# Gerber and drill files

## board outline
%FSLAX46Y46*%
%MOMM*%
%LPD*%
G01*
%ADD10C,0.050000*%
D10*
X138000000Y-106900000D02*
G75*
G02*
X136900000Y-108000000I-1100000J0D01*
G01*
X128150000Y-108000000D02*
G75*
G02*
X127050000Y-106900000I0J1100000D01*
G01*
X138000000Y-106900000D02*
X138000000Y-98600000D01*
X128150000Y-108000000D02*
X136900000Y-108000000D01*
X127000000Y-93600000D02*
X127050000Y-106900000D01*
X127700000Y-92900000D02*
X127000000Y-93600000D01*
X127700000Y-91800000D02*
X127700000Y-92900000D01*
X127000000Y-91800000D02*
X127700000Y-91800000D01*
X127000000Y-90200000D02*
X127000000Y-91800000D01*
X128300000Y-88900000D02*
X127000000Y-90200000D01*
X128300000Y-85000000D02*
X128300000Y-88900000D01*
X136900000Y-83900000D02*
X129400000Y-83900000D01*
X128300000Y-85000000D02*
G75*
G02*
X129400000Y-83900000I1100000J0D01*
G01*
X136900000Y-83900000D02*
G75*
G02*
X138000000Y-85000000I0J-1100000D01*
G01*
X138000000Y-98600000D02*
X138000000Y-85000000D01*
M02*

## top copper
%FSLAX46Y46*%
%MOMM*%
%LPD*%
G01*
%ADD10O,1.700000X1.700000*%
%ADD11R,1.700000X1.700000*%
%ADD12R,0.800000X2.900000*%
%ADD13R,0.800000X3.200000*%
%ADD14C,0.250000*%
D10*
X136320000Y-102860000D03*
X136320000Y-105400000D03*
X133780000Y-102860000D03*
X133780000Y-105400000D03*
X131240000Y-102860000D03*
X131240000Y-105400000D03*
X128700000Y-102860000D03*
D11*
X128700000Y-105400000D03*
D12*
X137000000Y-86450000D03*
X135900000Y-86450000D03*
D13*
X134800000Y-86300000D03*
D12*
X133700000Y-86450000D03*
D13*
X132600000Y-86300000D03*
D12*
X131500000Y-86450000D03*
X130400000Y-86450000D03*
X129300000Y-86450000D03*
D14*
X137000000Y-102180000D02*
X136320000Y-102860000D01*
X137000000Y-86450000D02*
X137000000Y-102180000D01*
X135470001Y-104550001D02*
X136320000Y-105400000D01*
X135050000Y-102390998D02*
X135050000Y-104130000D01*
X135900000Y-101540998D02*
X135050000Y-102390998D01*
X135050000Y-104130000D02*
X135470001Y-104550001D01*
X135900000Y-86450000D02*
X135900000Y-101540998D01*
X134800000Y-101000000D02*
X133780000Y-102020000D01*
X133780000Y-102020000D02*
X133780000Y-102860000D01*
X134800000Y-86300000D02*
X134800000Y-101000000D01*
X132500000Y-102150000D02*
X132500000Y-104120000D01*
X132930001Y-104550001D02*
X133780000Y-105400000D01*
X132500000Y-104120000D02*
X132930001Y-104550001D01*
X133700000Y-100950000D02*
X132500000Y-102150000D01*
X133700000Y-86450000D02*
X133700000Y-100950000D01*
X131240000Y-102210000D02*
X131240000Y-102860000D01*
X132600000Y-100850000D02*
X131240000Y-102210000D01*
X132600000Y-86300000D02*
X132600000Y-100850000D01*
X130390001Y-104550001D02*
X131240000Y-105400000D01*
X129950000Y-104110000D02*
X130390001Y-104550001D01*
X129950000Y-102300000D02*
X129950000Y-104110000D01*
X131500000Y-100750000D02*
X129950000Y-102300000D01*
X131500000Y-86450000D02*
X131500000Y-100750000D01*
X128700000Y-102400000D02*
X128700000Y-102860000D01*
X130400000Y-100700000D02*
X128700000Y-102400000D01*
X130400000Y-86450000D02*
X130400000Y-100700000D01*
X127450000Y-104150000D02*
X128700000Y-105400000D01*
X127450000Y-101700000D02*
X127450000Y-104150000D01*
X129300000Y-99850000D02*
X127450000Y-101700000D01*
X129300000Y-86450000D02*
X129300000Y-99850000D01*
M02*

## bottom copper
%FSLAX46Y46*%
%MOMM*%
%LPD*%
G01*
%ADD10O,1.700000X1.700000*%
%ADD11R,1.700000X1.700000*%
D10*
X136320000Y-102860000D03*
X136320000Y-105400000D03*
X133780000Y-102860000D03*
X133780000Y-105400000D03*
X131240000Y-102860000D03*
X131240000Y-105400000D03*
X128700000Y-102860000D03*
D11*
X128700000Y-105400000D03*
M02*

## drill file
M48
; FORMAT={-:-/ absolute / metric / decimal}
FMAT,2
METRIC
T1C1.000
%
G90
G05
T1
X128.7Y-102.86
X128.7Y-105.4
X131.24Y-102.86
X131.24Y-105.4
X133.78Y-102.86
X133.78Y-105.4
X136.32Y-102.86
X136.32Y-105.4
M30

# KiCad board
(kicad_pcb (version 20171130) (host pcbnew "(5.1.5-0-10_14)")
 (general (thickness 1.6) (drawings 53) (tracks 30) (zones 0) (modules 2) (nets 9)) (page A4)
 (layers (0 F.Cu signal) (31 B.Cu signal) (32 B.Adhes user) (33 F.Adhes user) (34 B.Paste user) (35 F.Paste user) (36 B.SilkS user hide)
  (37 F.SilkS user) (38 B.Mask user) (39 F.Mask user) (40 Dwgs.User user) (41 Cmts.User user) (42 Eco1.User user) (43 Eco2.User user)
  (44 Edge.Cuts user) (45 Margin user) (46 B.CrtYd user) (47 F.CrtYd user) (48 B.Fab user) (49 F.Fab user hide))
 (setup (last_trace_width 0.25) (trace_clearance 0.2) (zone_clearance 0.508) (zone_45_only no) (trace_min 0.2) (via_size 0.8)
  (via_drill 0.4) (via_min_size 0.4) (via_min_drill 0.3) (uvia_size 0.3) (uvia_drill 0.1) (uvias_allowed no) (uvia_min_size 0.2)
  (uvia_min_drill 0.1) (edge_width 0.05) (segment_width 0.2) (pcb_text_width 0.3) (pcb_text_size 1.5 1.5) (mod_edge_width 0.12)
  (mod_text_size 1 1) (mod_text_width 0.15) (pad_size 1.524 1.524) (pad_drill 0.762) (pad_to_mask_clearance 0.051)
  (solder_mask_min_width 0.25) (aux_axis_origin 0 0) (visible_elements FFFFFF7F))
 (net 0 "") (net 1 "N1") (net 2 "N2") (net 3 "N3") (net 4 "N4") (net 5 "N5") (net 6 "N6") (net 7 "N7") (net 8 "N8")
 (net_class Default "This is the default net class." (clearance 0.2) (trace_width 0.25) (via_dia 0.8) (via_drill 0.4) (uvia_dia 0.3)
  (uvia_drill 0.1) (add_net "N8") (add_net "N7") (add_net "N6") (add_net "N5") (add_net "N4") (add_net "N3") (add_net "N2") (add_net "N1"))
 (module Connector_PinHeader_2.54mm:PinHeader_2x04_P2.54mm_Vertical (layer F.Cu) (at 128.7 105.4 90)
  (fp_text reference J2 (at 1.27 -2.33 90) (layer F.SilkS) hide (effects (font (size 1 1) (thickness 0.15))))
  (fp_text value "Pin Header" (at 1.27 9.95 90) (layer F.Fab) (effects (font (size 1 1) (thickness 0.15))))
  (pad 8 thru_hole oval (at 2.54 7.62 90) (size 1.7 1.7) (drill 1) (layers *.Cu *.Mask) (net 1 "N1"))
  (pad 7 thru_hole oval (at 0 7.62 90) (size 1.7 1.7) (drill 1) (layers *.Cu *.Mask) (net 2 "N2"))
  (pad 6 thru_hole oval (at 2.54 5.08 90) (size 1.7 1.7) (drill 1) (layers *.Cu *.Mask) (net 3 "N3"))
  (pad 5 thru_hole oval (at 0 5.08 90) (size 1.7 1.7) (drill 1) (layers *.Cu *.Mask) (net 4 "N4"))
  (pad 4 thru_hole oval (at 2.54 2.54 90) (size 1.7 1.7) (drill 1) (layers *.Cu *.Mask) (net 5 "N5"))
  (pad 3 thru_hole oval (at 0 2.54 90) (size 1.7 1.7) (drill 1) (layers *.Cu *.Mask) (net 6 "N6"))
  (pad 2 thru_hole oval (at 2.54 0 90) (size 1.7 1.7) (drill 1) (layers *.Cu *.Mask) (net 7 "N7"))
  (pad 1 thru_hole rect (at 0 0 90) (size 1.7 1.7) (drill 1) (layers *.Cu *.Mask) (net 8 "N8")))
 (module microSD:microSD (layer F.Cu) (at 133.15 88)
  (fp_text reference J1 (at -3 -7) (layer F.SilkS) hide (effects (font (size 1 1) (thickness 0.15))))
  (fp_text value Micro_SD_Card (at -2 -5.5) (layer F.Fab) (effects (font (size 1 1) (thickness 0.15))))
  (pad 8 smd rect (at 3.85 -1.55) (size 0.8 2.9) (layers F.Cu F.Paste F.Mask) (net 1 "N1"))
  (pad 7 smd rect (at 2.75 -1.55) (size 0.8 2.9) (layers F.Cu F.Paste F.Mask) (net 2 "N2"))
  (pad 6 smd rect (at 1.65 -1.7) (size 0.8 3.2) (layers F.Cu F.Paste F.Mask) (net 3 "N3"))
  (pad 5 smd rect (at 0.55 -1.55) (size 0.8 2.9) (layers F.Cu F.Paste F.Mask) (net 4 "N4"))
  (pad 4 smd rect (at -0.55 -1.7) (size 0.8 3.2) (layers F.Cu F.Paste F.Mask) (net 5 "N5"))
  (pad 3 smd rect (at -1.65 -1.55) (size 0.8 2.9) (layers F.Cu F.Paste F.Mask) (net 6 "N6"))
  (pad 2 smd rect (at -2.75 -1.55) (size 0.8 2.9) (layers F.Cu F.Paste F.Mask) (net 7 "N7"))
  (pad 1 smd rect (at -3.85 -1.55) (size 0.8 2.9) (layers F.Cu F.Paste F.Mask) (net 8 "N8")))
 (gr_arc (start 136.9 106.9) (end 136.9 108) (angle -90) (layer Edge.Cuts) (width 0.05))
 (gr_arc (start 128.15 106.9) (end 127.05 106.9) (angle -90) (layer Edge.Cuts) (width 0.05))
 (gr_line (start 138 106.9) (end 138 98.6) (layer Edge.Cuts) (width 0.05))
 (gr_line (start 128.15 108) (end 136.9 108) (layer Edge.Cuts) (width 0.05))
 (gr_line (start 127 93.6) (end 127.05 106.9) (layer Edge.Cuts) (width 0.05))
 (gr_line (start 127.7 92.9) (end 127 93.6) (layer Edge.Cuts) (width 0.05))
 (gr_line (start 127.7 91.8) (end 127.7 92.9) (layer Edge.Cuts) (width 0.05))
 (gr_line (start 127 91.8) (end 127.7 91.8) (layer Edge.Cuts) (width 0.05))
 (gr_line (start 127 90.2) (end 127 91.8) (layer Edge.Cuts) (width 0.05))
 (gr_line (start 128.3 88.9) (end 127 90.2) (layer Edge.Cuts) (width 0.05))
 (gr_line (start 128.3 85) (end 128.3 88.9) (layer Edge.Cuts) (width 0.05))
 (gr_line (start 136.9 83.9) (end 129.4 83.9) (layer Edge.Cuts) (width 0.05))
 (gr_arc (start 129.4 85) (end 129.4 83.9) (angle -90) (layer Edge.Cuts) (width 0.05))
 (gr_arc (start 136.9 85) (end 138 85) (angle -90) (layer Edge.Cuts) (width 0.05))
 (gr_line (start 138 98.6) (end 138 85) (layer Edge.Cuts) (width 0.05))
 (segment (start 137 102.18) (end 136.32 102.86) (width 0.25) (layer F.Cu) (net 1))
 (segment (start 137 86.45) (end 137 102.18) (width 0.25) (layer F.Cu) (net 1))
 (segment (start 135.470001 104.550001) (end 136.32 105.4) (width 0.25) (layer F.Cu) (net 2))
 (segment (start 135.05 102.390998) (end 135.05 104.13) (width 0.25) (layer F.Cu) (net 2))
 (segment (start 135.9 101.540998) (end 135.05 102.390998) (width 0.25) (layer F.Cu) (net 2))
 (segment (start 135.05 104.13) (end 135.470001 104.550001) (width 0.25) (layer F.Cu) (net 2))
 (segment (start 135.9 86.45) (end 135.9 101.540998) (width 0.25) (layer F.Cu) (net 2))
 (segment (start 134.8 101) (end 133.78 102.02) (width 0.25) (layer F.Cu) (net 3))
 (segment (start 133.78 102.02) (end 133.78 102.86) (width 0.25) (layer F.Cu) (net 3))
 (segment (start 134.8 86.3) (end 134.8 101) (width 0.25) (layer F.Cu) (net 3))
 (segment (start 132.5 102.15) (end 132.5 104.12) (width 0.25) (layer F.Cu) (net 4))
 (segment (start 132.930001 104.550001) (end 133.78 105.4) (width 0.25) (layer F.Cu) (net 4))
 (segment (start 132.5 104.12) (end 132.930001 104.550001) (width 0.25) (layer F.Cu) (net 4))
 (segment (start 133.7 100.95) (end 132.5 102.15) (width 0.25) (layer F.Cu) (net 4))
 (segment (start 133.7 86.45) (end 133.7 100.95) (width 0.25) (layer F.Cu) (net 4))
 (segment (start 131.24 102.21) (end 131.24 102.86) (width 0.25) (layer F.Cu) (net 5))
 (segment (start 132.6 100.85) (end 131.24 102.21) (width 0.25) (layer F.Cu) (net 5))
 (segment (start 132.6 86.3) (end 132.6 100.85) (width 0.25) (layer F.Cu) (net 5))
 (segment (start 130.390001 104.550001) (end 131.24 105.4) (width 0.25) (layer F.Cu) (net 6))
 (segment (start 129.95 104.11) (end 130.390001 104.550001) (width 0.25) (layer F.Cu) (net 6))
 (segment (start 129.95 102.3) (end 129.95 104.11) (width 0.25) (layer F.Cu) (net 6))
 (segment (start 131.5 100.75) (end 129.95 102.3) (width 0.25) (layer F.Cu) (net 6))
 (segment (start 131.5 86.45) (end 131.5 100.75) (width 0.25) (layer F.Cu) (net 6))
 (segment (start 128.7 102.4) (end 128.7 102.86) (width 0.25) (layer F.Cu) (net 7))
 (segment (start 130.4 100.7) (end 128.7 102.4) (width 0.25) (layer F.Cu) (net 7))
 (segment (start 130.4 86.45) (end 130.4 100.7) (width 0.25) (layer F.Cu) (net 7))
 (segment (start 127.45 104.15) (end 128.7 105.4) (width 0.25) (layer F.Cu) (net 8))
 (segment (start 127.45 101.7) (end 127.45 104.15) (width 0.25) (layer F.Cu) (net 8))
 (segment (start 129.3 99.85) (end 127.45 101.7) (width 0.25) (layer F.Cu) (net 8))
 (segment (start 129.3 86.45) (end 129.3 99.85) (width 0.25) (layer F.Cu) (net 8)))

